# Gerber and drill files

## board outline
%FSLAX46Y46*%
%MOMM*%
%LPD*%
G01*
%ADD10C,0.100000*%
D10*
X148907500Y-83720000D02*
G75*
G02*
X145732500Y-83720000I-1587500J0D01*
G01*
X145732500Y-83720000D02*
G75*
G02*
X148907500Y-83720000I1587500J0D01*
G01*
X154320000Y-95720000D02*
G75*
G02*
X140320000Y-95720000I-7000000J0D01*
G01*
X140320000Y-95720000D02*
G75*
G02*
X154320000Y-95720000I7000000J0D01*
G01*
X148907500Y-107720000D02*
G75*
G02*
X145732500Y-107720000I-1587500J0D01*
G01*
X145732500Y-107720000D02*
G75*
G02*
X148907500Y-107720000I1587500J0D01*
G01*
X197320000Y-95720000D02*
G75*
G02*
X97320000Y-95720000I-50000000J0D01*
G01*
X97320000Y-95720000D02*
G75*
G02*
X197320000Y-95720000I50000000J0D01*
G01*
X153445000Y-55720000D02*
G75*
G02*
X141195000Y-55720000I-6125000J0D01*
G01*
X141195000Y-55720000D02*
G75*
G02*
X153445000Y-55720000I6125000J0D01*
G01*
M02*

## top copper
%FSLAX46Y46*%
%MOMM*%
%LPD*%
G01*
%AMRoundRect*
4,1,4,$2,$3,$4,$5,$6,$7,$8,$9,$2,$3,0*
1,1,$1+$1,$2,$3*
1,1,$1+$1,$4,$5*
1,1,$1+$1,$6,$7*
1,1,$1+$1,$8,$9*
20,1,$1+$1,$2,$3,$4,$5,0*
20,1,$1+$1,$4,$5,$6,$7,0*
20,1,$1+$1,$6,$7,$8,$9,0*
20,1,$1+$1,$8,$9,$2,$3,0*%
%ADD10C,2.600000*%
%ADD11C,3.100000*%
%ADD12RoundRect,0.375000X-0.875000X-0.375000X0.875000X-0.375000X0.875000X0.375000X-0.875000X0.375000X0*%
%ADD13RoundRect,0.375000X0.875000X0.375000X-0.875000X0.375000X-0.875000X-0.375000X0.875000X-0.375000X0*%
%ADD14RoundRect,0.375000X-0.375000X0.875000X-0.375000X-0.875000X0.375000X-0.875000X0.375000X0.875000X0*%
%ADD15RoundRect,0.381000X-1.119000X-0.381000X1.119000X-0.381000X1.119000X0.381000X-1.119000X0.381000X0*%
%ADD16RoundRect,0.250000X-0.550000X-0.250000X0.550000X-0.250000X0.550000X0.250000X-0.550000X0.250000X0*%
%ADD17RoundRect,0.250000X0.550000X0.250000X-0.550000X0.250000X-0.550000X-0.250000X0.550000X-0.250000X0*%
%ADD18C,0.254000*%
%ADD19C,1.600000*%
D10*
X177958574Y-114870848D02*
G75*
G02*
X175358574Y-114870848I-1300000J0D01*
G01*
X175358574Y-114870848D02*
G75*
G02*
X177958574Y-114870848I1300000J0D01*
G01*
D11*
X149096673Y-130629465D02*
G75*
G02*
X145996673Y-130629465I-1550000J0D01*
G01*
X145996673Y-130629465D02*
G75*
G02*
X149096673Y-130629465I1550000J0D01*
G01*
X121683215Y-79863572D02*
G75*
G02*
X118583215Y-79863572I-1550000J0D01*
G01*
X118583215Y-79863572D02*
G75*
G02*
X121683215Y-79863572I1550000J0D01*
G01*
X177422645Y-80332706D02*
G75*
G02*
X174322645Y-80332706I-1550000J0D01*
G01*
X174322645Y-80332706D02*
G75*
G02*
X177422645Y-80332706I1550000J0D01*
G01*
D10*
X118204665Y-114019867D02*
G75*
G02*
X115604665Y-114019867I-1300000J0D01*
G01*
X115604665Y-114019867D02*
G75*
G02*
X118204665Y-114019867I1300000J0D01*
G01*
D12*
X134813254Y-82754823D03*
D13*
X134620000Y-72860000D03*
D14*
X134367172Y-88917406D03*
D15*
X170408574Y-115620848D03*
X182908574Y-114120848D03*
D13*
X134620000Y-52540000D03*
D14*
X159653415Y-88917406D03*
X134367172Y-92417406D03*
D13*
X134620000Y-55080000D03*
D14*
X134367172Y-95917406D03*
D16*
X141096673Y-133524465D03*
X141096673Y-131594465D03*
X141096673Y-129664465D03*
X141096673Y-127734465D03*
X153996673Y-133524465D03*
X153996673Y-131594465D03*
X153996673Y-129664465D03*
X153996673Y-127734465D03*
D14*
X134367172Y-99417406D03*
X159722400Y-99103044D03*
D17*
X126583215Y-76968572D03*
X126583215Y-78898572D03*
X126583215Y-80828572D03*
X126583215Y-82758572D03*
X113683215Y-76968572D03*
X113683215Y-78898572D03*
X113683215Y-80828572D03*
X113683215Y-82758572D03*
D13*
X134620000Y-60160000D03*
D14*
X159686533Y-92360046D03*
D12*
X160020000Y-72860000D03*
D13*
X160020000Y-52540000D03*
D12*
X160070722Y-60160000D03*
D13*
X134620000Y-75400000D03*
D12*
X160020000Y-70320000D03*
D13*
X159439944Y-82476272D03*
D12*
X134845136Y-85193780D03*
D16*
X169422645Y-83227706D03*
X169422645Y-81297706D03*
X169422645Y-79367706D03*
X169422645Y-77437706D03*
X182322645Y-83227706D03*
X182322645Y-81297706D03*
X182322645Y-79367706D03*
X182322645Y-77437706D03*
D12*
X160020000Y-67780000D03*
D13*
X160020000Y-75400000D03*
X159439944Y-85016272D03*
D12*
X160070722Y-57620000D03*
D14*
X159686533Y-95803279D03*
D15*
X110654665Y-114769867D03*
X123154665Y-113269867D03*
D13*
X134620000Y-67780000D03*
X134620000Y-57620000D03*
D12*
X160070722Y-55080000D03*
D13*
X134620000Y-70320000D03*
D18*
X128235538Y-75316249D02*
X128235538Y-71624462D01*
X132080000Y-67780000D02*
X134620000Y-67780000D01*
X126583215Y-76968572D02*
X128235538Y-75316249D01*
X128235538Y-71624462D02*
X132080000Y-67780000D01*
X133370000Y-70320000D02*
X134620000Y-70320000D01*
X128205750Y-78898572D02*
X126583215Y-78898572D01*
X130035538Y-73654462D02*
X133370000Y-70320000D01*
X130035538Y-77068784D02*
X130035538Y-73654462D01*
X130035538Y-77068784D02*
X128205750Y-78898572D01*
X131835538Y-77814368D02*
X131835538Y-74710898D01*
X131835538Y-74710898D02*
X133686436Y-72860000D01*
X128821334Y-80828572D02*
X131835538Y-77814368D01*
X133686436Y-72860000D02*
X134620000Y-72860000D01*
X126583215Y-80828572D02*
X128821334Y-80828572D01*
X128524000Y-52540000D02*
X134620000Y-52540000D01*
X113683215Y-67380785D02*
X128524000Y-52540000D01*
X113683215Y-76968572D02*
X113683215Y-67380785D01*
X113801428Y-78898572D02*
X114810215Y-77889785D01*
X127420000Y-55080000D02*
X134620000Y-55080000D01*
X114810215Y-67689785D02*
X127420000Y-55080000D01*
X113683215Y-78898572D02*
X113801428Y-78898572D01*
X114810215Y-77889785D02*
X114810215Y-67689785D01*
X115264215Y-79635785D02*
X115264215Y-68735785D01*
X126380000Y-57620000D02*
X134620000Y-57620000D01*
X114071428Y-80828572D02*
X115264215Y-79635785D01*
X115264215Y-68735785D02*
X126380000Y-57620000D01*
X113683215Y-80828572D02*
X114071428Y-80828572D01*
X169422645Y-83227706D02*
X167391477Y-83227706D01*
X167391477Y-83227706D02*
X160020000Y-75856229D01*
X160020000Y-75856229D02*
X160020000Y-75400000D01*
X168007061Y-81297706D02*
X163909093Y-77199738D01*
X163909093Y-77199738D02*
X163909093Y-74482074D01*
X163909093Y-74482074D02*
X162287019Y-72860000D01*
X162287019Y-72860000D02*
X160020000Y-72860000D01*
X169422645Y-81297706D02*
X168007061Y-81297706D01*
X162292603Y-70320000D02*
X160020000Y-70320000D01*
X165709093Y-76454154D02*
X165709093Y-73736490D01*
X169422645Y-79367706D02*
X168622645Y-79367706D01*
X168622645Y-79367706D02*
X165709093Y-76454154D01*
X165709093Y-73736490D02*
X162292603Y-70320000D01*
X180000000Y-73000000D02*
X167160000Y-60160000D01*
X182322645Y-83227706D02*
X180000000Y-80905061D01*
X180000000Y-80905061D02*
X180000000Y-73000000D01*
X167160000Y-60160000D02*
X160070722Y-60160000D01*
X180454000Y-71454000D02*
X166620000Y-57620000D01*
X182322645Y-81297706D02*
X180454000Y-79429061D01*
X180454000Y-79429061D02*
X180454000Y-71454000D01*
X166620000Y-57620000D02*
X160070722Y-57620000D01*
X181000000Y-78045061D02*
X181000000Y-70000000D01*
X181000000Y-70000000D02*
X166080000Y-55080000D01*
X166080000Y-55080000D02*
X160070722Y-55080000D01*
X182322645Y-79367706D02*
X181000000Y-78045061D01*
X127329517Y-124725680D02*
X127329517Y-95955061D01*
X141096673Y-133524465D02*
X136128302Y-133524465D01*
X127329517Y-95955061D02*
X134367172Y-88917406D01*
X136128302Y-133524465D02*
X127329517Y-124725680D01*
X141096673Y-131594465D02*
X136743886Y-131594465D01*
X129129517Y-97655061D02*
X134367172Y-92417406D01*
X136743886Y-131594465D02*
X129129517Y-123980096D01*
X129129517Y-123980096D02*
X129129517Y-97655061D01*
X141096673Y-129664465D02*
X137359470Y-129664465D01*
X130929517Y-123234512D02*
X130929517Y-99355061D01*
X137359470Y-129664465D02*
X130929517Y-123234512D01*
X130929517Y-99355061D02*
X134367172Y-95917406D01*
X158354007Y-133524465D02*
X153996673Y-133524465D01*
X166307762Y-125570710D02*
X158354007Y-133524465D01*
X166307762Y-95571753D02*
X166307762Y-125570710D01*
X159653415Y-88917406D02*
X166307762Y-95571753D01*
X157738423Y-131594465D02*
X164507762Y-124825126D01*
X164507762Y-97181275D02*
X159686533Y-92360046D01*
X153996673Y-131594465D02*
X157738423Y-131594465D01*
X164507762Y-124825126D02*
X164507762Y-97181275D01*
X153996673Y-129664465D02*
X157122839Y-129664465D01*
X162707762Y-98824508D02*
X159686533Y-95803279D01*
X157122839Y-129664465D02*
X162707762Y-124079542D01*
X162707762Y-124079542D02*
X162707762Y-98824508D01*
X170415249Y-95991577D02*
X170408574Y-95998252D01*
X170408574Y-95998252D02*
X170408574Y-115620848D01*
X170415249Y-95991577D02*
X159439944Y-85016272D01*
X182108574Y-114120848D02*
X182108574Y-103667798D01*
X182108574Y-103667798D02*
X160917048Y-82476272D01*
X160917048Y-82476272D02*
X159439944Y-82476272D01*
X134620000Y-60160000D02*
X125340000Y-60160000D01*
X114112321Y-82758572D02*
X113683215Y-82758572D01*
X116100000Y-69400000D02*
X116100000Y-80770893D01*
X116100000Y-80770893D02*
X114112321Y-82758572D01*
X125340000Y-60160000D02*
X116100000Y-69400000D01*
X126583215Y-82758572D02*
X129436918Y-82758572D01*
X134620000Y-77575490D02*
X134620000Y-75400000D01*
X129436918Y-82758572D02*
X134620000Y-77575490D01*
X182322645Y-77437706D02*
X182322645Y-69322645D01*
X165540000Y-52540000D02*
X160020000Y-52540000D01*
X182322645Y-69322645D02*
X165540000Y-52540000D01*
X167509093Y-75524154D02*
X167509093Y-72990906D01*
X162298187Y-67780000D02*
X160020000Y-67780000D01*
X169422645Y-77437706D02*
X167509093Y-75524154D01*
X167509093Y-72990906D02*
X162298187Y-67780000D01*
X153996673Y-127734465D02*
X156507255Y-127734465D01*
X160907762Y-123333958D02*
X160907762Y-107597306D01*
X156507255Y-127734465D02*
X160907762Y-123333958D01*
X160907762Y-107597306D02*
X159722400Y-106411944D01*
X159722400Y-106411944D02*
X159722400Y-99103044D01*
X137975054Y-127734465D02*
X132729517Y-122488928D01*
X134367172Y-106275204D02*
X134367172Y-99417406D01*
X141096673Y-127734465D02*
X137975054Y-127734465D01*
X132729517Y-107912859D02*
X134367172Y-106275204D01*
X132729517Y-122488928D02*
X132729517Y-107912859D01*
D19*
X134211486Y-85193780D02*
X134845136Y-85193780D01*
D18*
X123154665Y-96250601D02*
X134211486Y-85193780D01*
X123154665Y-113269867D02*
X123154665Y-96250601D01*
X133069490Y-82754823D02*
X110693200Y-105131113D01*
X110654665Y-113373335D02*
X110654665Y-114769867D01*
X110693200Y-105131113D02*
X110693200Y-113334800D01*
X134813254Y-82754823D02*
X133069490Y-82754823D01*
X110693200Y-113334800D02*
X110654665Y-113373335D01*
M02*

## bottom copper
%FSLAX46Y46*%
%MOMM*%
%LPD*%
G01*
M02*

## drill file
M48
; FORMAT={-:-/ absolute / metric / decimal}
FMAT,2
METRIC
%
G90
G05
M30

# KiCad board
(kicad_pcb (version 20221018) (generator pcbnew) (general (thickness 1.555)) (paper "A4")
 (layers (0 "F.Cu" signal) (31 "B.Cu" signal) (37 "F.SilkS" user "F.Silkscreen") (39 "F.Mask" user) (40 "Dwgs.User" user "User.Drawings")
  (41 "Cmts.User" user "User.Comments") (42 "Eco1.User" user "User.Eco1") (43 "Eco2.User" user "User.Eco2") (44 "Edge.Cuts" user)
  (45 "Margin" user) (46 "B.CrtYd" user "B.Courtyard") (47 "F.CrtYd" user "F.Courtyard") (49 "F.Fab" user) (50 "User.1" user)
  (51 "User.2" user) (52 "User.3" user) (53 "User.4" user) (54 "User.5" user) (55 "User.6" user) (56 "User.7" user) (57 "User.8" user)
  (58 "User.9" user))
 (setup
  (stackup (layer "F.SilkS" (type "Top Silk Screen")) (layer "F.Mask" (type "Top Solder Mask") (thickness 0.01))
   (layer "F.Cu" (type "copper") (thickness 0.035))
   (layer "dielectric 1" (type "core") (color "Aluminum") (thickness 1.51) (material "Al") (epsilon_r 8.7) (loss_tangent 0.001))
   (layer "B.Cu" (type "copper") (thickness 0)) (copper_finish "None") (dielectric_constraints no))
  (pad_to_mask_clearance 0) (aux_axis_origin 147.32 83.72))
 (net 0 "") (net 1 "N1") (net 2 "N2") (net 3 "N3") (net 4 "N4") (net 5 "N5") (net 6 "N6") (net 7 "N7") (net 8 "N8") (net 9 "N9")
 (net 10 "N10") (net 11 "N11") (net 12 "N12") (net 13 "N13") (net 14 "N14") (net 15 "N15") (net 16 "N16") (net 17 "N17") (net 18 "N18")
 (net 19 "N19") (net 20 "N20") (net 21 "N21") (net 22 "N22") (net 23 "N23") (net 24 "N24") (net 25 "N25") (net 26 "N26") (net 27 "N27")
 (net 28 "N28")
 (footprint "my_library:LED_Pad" (layer "F.Cu") (at 134.813254 85.294823)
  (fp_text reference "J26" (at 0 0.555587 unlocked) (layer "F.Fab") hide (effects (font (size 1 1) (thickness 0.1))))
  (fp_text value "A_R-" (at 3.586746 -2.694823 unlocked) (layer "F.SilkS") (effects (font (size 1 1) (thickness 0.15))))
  (pad "1" smd roundrect (at 0 -2.54) (size 2.5 1.5) (layers "F.Cu" "F.Mask") (roundrect_rratio 0.25) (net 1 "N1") (thermal_bridge_angle 45)))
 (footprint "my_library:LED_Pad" (layer "F.Cu") (at 134.62 70.32 180)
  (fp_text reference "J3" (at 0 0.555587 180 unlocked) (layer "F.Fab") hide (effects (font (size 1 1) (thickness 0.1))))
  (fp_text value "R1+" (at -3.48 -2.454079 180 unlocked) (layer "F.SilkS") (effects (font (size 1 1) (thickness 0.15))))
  (pad "1" smd roundrect (at 0 -2.54 180) (size 2.5 1.5) (layers "F.Cu" "F.Mask") (roundrect_rratio 0.25) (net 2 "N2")
   (thermal_bridge_angle 45)))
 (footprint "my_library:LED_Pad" (layer "F.Cu") (at 131.827172 88.917406 -90)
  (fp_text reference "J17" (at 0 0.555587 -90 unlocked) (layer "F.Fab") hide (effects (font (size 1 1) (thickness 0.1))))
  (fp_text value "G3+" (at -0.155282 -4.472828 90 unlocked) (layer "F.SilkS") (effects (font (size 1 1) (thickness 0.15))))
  (pad "1" smd roundrect (at 0 -2.54 270) (size 2.5 1.5) (layers "F.Cu" "F.Mask") (roundrect_rratio 0.25) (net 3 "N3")
   (thermal_bridge_angle 45)))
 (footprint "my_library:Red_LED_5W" (layer "F.Cu") (at 177.028574 114.120848)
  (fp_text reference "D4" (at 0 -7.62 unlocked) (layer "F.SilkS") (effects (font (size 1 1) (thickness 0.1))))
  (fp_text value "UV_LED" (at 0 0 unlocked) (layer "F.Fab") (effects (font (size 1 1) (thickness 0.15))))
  (fp_circle (center -0.37 0.75) (end 2.13 0.75) (stroke (width 0.2) (type solid)) (fill solid) (layer "F.Cu"))
  (pad "1" smd roundrect (at -6.62 1.5) (size 3 1.524) (layers "F.Cu" "F.Paste" "F.Mask") (roundrect_rratio 0.25) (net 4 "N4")
   (thermal_bridge_angle 45))
  (pad "2" smd roundrect (at 5.88 0) (size 3 1.524) (layers "F.Cu" "F.Paste" "F.Mask") (roundrect_rratio 0.25) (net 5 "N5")
   (thermal_bridge_angle 45)))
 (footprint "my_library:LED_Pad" (layer "F.Cu") (at 134.62 50 180)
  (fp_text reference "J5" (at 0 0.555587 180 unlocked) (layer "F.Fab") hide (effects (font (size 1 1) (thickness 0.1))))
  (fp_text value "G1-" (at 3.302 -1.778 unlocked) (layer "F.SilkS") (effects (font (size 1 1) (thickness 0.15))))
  (pad "1" smd roundrect (at 0 -2.54 180) (size 2.5 1.5) (layers "F.Cu" "F.Mask") (roundrect_rratio 0.25) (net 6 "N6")
   (thermal_bridge_angle 45)))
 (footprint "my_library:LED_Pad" (layer "F.Cu") (at 157.113415 88.917406 -90)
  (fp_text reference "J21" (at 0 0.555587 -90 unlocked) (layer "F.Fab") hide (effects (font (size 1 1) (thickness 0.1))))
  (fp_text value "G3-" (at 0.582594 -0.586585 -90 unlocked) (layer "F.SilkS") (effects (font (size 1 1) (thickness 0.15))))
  (pad "1" smd roundrect (at 0 -2.54 270) (size 2.5 1.5) (layers "F.Cu" "F.Mask") (roundrect_rratio 0.25) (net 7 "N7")
   (thermal_bridge_angle 45)))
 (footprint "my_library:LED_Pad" (layer "F.Cu") (at 131.827172 92.417406 -90)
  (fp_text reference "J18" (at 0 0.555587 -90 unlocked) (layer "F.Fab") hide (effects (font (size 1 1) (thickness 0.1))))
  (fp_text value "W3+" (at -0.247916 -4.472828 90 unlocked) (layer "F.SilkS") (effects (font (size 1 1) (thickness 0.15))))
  (pad "1" smd roundrect (at 0 -2.54 270) (size 2.5 1.5) (layers "F.Cu" "F.Mask") (roundrect_rratio 0.25) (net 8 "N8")
   (thermal_bridge_angle 45)))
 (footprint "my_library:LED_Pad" (layer "F.Cu") (at 134.62 52.54 180)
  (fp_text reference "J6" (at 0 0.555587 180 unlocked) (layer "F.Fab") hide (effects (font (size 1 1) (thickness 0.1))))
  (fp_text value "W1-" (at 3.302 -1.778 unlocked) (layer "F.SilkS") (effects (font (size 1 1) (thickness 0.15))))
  (pad "1" smd roundrect (at 0 -2.54 180) (size 2.5 1.5) (layers "F.Cu" "F.Mask") (roundrect_rratio 0.25) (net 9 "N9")
   (thermal_bridge_angle 45)))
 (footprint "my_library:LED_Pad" (layer "F.Cu") (at 131.827172 95.917406 -90)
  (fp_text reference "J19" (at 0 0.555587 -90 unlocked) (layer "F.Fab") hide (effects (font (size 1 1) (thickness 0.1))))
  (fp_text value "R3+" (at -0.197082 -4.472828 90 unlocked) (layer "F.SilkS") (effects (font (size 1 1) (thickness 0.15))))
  (pad "1" smd roundrect (at 0 -2.54 270) (size 2.5 1.5) (layers "F.Cu" "F.Mask") (roundrect_rratio 0.25) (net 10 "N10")
   (thermal_bridge_angle 45)))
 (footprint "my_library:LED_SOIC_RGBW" (layer "F.Cu") (at 145.916673 139.214465)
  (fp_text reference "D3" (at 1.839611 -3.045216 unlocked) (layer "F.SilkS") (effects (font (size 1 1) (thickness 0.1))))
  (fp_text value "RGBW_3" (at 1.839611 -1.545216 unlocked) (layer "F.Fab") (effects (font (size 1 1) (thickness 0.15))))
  (fp_circle (center 1.63 -8.585) (end 4.63 -8.585) (stroke (width 0.2) (type solid)) (fill solid) (layer "F.Cu"))
  (pad "1" smd roundrect (at -4.82 -5.69) (size 1.6 1) (layers "F.Cu" "F.Mask") (roundrect_rratio 0.25) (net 3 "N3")
   (thermal_bridge_angle 45))
  (pad "2" smd roundrect (at -4.82 -7.62) (size 1.6 1) (layers "F.Cu" "F.Mask") (roundrect_rratio 0.25) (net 8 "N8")
   (thermal_bridge_angle 45))
  (pad "3" smd roundrect (at -4.82 -9.55) (size 1.6 1) (layers "F.Cu" "F.Mask") (roundrect_rratio 0.25) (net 10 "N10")
   (thermal_bridge_angle 45))
  (pad "4" smd roundrect (at -4.82 -11.48) (size 1.6 1) (layers "F.Cu" "F.Mask") (roundrect_rratio 0.25) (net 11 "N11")
   (thermal_bridge_angle 45))
  (pad "5" smd roundrect (at 8.08 -5.69) (size 1.6 1) (layers "F.Cu" "F.Mask") (roundrect_rratio 0.25) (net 7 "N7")
   (thermal_bridge_angle 45))
  (pad "6" smd roundrect (at 8.08 -7.62) (size 1.6 1) (layers "F.Cu" "F.Mask") (roundrect_rratio 0.25) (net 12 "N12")
   (thermal_bridge_angle 45))
  (pad "7" smd roundrect (at 8.08 -9.55) (size 1.6 1) (layers "F.Cu" "F.Mask") (roundrect_rratio 0.25) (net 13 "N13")
   (thermal_bridge_angle 45))
  (pad "8" smd roundrect (at 8.08 -11.48) (size 1.6 1) (layers "F.Cu" "F.Mask") (roundrect_rratio 0.25) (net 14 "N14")
   (thermal_bridge_angle 45)))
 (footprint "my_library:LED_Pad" (layer "F.Cu") (at 131.827172 99.417406 -90)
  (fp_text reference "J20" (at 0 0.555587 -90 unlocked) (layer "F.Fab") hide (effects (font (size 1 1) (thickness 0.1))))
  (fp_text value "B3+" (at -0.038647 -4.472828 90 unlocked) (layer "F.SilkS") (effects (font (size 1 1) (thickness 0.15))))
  (pad "1" smd roundrect (at 0 -2.54 270) (size 2.5 1.5) (layers "F.Cu" "F.Mask") (roundrect_rratio 0.25) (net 11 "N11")
   (thermal_bridge_angle 45)))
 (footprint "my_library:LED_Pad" (layer "F.Cu") (at 157.1824 99.103044 -90)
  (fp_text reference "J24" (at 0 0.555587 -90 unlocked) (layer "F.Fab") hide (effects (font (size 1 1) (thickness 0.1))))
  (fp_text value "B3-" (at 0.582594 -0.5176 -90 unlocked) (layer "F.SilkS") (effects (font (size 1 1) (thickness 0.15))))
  (pad "1" smd roundrect (at 0 -2.54 270) (size 2.5 1.5) (layers "F.Cu" "F.Mask") (roundrect_rratio 0.25) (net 14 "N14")
   (thermal_bridge_angle 45)))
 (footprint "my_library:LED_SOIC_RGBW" (layer "F.Cu") (at 121.763215 71.278572 180)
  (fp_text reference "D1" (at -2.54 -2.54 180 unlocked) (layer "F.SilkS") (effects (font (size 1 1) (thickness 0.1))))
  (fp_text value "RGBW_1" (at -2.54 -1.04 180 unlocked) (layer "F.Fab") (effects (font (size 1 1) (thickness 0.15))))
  (fp_circle (center 1.63 -8.585) (end 4.63 -8.585) (stroke (width 0.2) (type solid)) (fill solid) (layer "F.Cu"))
  (pad "1" smd roundrect (at -4.82 -5.69 180) (size 1.6 1) (layers "F.Cu" "F.Mask") (roundrect_rratio 0.25) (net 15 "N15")
   (thermal_bridge_angle 45))
  (pad "2" smd roundrect (at -4.82 -7.62 180) (size 1.6 1) (layers "F.Cu" "F.Mask") (roundrect_rratio 0.25) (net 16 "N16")
   (thermal_bridge_angle 45))
  (pad "3" smd roundrect (at -4.82 -9.55 180) (size 1.6 1) (layers "F.Cu" "F.Mask") (roundrect_rratio 0.25) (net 2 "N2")
   (thermal_bridge_angle 45))
  (pad "4" smd roundrect (at -4.82 -11.48 180) (size 1.6 1) (layers "F.Cu" "F.Mask") (roundrect_rratio 0.25) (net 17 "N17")
   (thermal_bridge_angle 45))
  (pad "5" smd roundrect (at 8.08 -5.69 180) (size 1.6 1) (layers "F.Cu" "F.Mask") (roundrect_rratio 0.25) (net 6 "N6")
   (thermal_bridge_angle 45))
  (pad "6" smd roundrect (at 8.08 -7.62 180) (size 1.6 1) (layers "F.Cu" "F.Mask") (roundrect_rratio 0.25) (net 9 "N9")
   (thermal_bridge_angle 45))
  (pad "7" smd roundrect (at 8.08 -9.55 180) (size 1.6 1) (layers "F.Cu" "F.Mask") (roundrect_rratio 0.25) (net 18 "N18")
   (thermal_bridge_angle 45))
  (pad "8" smd roundrect (at 8.08 -11.48 180) (size 1.6 1) (layers "F.Cu" "F.Mask") (roundrect_rratio 0.25) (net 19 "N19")
   (thermal_bridge_angle 45)))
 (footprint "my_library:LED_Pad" (layer "F.Cu") (at 134.62 57.62 180)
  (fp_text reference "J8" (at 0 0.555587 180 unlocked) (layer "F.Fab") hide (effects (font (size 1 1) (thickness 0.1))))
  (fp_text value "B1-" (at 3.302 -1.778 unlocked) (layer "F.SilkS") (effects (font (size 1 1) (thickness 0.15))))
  (pad "1" smd roundrect (at 0 -2.54 180) (size 2.5 1.5) (layers "F.Cu" "F.Mask") (roundrect_rratio 0.25) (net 19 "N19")
   (thermal_bridge_angle 45)))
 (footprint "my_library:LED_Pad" (layer "F.Cu") (at 157.146533 92.360046 -90)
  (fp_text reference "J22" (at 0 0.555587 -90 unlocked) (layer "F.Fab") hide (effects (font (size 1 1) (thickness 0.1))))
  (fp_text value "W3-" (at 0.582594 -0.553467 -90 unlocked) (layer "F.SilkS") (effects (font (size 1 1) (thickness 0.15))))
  (pad "1" smd roundrect (at 0 -2.54 270) (size 2.5 1.5) (layers "F.Cu" "F.Mask") (roundrect_rratio 0.25) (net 12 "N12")
   (thermal_bridge_angle 45)))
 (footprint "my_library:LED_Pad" (layer "F.Cu") (at 160.02 75.4)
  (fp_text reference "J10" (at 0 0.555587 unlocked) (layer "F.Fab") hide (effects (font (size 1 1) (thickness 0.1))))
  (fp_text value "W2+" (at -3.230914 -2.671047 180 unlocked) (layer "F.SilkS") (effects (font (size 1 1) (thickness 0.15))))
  (pad "1" smd roundrect (at 0 -2.54) (size 2.5 1.5) (layers "F.Cu" "F.Mask") (roundrect_rratio 0.25) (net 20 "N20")
   (thermal_bridge_angle 45)))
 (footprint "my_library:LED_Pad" (layer "F.Cu") (at 160.02 50 180)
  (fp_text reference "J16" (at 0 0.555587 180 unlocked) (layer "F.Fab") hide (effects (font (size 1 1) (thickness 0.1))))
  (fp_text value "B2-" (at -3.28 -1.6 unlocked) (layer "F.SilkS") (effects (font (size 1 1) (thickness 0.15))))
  (pad "1" smd roundrect (at 0 -2.54 180) (size 2.5 1.5) (layers "F.Cu" "F.Mask") (roundrect_rratio 0.25) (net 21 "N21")
   (thermal_bridge_angle 45)))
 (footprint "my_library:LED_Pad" (layer "F.Cu") (at 160.070722 62.7)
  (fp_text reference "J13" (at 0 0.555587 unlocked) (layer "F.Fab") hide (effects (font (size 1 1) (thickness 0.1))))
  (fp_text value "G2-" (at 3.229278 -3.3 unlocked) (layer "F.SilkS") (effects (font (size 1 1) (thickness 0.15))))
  (pad "1" smd roundrect (at 0 -2.54) (size 2.5 1.5) (layers "F.Cu" "F.Mask") (roundrect_rratio 0.25) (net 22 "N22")
   (thermal_bridge_angle 45)))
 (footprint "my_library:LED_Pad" (layer "F.Cu") (at 134.62 72.86 180)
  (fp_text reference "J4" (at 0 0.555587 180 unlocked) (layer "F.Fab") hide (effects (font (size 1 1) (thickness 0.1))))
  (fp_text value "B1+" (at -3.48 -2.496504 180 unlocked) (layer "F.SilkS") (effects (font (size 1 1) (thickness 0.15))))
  (pad "1" smd roundrect (at 0 -2.54 180) (size 2.5 1.5) (layers "F.Cu" "F.Mask") (roundrect_rratio 0.25) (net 17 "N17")
   (thermal_bridge_angle 45)))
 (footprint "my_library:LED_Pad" (layer "F.Cu") (at 160.02 72.86)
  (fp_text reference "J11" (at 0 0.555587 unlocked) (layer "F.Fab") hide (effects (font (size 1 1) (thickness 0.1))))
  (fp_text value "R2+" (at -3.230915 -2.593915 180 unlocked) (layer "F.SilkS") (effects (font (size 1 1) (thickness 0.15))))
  (pad "1" smd roundrect (at 0 -2.54) (size 2.5 1.5) (layers "F.Cu" "F.Mask") (roundrect_rratio 0.25) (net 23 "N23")
   (thermal_bridge_angle 45)))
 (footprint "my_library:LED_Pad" (layer "F.Cu") (at 159.439944 79.936272 180)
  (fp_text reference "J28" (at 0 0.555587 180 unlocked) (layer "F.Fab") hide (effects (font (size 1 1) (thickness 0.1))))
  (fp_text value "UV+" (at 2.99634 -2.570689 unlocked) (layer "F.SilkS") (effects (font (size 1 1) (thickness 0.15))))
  (pad "1" smd roundrect (at 0 -2.54 180) (size 2.5 1.5) (layers "F.Cu" "F.Mask") (roundrect_rratio 0.25) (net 5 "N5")
   (thermal_bridge_angle 45)))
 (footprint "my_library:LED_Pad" (layer "F.Cu") (at 134.845136 87.73378)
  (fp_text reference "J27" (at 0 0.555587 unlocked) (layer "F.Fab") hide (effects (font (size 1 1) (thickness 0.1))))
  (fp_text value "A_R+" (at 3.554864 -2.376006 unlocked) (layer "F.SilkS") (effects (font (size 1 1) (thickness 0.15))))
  (pad "1" smd roundrect (at 0 -2.54) (size 2.5 1.5) (layers "F.Cu" "F.Mask") (roundrect_rratio 0.25) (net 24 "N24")
   (thermal_bridge_angle 45)))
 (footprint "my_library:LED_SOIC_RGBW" (layer "F.Cu") (at 174.242645 88.917706)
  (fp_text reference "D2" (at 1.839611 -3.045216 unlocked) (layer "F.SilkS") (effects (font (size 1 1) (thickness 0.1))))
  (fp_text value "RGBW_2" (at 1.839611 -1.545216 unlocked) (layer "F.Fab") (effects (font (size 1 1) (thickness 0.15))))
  (fp_circle (center 1.63 -8.585) (end 4.63 -8.585) (stroke (width 0.2) (type solid)) (fill solid) (layer "F.Cu"))
  (pad "1" smd roundrect (at -4.82 -5.69) (size 1.6 1) (layers "F.Cu" "F.Mask") (roundrect_rratio 0.25) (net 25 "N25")
   (thermal_bridge_angle 45))
  (pad "2" smd roundrect (at -4.82 -7.62) (size 1.6 1) (layers "F.Cu" "F.Mask") (roundrect_rratio 0.25) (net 20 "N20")
   (thermal_bridge_angle 45))
  (pad "3" smd roundrect (at -4.82 -9.55) (size 1.6 1) (layers "F.Cu" "F.Mask") (roundrect_rratio 0.25) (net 23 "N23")
   (thermal_bridge_angle 45))
  (pad "4" smd roundrect (at -4.82 -11.48) (size 1.6 1) (layers "F.Cu" "F.Mask") (roundrect_rratio 0.25) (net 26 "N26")
   (thermal_bridge_angle 45))
  (pad "5" smd roundrect (at 8.08 -5.69) (size 1.6 1) (layers "F.Cu" "F.Mask") (roundrect_rratio 0.25) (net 22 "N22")
   (thermal_bridge_angle 45))
  (pad "6" smd roundrect (at 8.08 -7.62) (size 1.6 1) (layers "F.Cu" "F.Mask") (roundrect_rratio 0.25) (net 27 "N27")
   (thermal_bridge_angle 45))
  (pad "7" smd roundrect (at 8.08 -9.55) (size 1.6 1) (layers "F.Cu" "F.Mask") (roundrect_rratio 0.25) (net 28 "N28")
   (thermal_bridge_angle 45))
  (pad "8" smd roundrect (at 8.08 -11.48) (size 1.6 1) (layers "F.Cu" "F.Mask") (roundrect_rratio 0.25) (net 21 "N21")
   (thermal_bridge_angle 45)))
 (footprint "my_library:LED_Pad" (layer "F.Cu") (at 160.02 70.32)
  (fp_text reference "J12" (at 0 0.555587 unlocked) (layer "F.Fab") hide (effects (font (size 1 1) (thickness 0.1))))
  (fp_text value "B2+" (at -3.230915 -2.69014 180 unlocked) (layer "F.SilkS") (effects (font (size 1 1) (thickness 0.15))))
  (pad "1" smd roundrect (at 0 -2.54) (size 2.5 1.5) (layers "F.Cu" "F.Mask") (roundrect_rratio 0.25) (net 26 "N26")
   (thermal_bridge_angle 45)))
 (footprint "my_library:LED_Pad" (layer "F.Cu") (at 160.02 72.86 180)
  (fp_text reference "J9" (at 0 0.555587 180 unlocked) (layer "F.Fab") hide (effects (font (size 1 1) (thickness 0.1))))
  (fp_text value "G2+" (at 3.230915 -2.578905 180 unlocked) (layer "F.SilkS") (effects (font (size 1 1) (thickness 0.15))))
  (pad "1" smd roundrect (at 0 -2.54 180) (size 2.5 1.5) (layers "F.Cu" "F.Mask") (roundrect_rratio 0.25) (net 25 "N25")
   (thermal_bridge_angle 45)))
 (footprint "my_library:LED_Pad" (layer "F.Cu") (at 159.439944 82.476272 180)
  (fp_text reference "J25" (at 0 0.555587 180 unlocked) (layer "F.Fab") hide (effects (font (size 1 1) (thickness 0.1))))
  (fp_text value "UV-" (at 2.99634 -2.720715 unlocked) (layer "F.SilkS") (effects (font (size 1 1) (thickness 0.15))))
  (pad "1" smd roundrect (at 0 -2.54 180) (size 2.5 1.5) (layers "F.Cu" "F.Mask") (roundrect_rratio 0.25) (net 4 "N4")
   (thermal_bridge_angle 45)))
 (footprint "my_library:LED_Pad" (layer "F.Cu") (at 160.070722 60.16)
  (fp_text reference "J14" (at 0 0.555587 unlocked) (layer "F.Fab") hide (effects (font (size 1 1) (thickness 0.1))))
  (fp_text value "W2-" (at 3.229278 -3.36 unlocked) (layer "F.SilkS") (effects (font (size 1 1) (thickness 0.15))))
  (pad "1" smd roundrect (at 0 -2.54) (size 2.5 1.5) (layers "F.Cu" "F.Mask") (roundrect_rratio 0.25) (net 27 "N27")
   (thermal_bridge_angle 45)))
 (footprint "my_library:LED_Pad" (layer "F.Cu") (at 157.146533 95.803279 -90)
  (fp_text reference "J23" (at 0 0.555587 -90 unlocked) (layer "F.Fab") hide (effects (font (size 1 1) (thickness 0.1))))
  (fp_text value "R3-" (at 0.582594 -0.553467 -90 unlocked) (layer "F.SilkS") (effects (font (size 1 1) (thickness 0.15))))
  (pad "1" smd roundrect (at 0 -2.54 270) (size 2.5 1.5) (layers "F.Cu" "F.Mask") (roundrect_rratio 0.25) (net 13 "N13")
   (thermal_bridge_angle 45)))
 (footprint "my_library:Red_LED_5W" (layer "F.Cu") (at 117.274665 113.269867)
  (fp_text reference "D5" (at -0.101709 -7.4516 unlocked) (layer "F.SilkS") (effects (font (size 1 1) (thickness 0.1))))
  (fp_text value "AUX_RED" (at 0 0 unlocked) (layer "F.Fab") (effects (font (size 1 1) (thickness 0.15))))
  (fp_circle (center -0.37 0.75) (end 2.13 0.75) (stroke (width 0.2) (type solid)) (fill solid) (layer "F.Cu"))
  (pad "1" smd roundrect (at -6.62 1.5) (size 3 1.524) (layers "F.Cu" "F.Paste" "F.Mask") (roundrect_rratio 0.25) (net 1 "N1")
   (thermal_bridge_angle 45))
  (pad "2" smd roundrect (at 5.88 0) (size 3 1.524) (layers "F.Cu" "F.Paste" "F.Mask") (roundrect_rratio 0.25) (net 24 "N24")
   (thermal_bridge_angle 45)))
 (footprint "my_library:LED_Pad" (layer "F.Cu") (at 134.62 65.24 180)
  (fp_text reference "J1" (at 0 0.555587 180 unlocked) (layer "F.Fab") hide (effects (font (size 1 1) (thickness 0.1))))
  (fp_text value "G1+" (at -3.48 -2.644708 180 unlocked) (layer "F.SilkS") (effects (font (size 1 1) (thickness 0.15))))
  (pad "1" smd roundrect (at 0 -2.54 180) (size 2.5 1.5) (layers "F.Cu" "F.Mask") (roundrect_rratio 0.25) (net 15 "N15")
   (thermal_bridge_angle 45)))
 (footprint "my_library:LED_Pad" (layer "F.Cu") (at 134.62 55.08 180)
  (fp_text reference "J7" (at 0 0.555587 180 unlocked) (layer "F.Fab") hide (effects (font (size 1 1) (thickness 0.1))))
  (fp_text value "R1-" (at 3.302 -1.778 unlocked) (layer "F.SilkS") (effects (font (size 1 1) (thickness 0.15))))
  (pad "1" smd roundrect (at 0 -2.54 180) (size 2.5 1.5) (layers "F.Cu" "F.Mask") (roundrect_rratio 0.25) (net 18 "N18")
   (thermal_bridge_angle 45)))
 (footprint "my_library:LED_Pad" (layer "F.Cu") (at 160.070722 57.62)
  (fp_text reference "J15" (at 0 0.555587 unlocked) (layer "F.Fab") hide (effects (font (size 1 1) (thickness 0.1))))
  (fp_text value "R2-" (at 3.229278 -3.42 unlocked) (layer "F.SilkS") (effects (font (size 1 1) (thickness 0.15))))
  (pad "1" smd roundrect (at 0 -2.54) (size 2.5 1.5) (layers "F.Cu" "F.Mask") (roundrect_rratio 0.25) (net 28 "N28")
   (thermal_bridge_angle 45)))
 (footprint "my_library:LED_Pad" (layer "F.Cu") (at 134.62 67.78 180)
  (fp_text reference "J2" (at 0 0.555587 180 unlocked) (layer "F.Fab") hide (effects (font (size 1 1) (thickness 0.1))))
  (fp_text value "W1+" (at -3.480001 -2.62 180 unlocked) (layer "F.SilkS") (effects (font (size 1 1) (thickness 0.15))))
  (pad "1" smd roundrect (at 0 -2.54 180) (size 2.5 1.5) (layers "F.Cu" "F.Mask") (roundrect_rratio 0.25) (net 16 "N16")
   (thermal_bridge_angle 45)))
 (gr_circle locked (center 147.32 83.72) (end 148.9075 83.72) (stroke (width 0.1) (type default)) (fill none) (layer "Edge.Cuts"))
 (gr_circle locked (center 147.32 95.72) (end 154.32 95.72) (stroke (width 0.1) (type default)) (fill none) (layer "Edge.Cuts"))
 (gr_circle locked (center 147.32 107.72) (end 148.9075 107.72) (stroke (width 0.1) (type default)) (fill none) (layer "Edge.Cuts"))
 (gr_circle locked (center 147.32 95.72) (end 197.32 95.72) (stroke (width 0.1) (type default)) (fill none) (layer "Edge.Cuts"))
 (gr_circle locked (center 147.32 55.72) (end 153.445 55.72) (stroke (width 0.1) (type default)) (fill none) (layer "Edge.Cuts"))
 (segment (start 128.235538 75.316249) (end 128.235538 71.624462) (width 0.254) (layer "F.Cu") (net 15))
 (segment (start 132.08 67.78) (end 134.62 67.78) (width 0.254) (layer "F.Cu") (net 15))
 (segment (start 126.583215 76.968572) (end 128.235538 75.316249) (width 0.254) (layer "F.Cu") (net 15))
 (segment (start 128.235538 71.624462) (end 132.08 67.78) (width 0.254) (layer "F.Cu") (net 15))
 (segment (start 133.37 70.32) (end 134.62 70.32) (width 0.254) (layer "F.Cu") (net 16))
 (segment (start 128.20575 78.898572) (end 126.583215 78.898572) (width 0.254) (layer "F.Cu") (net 16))
 (segment (start 130.035538 73.654462) (end 133.37 70.32) (width 0.254) (layer "F.Cu") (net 16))
 (segment (start 130.035538 77.068784) (end 130.035538 73.654462) (width 0.254) (layer "F.Cu") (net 16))
 (segment (start 130.035538 77.068784) (end 128.20575 78.898572) (width 0.254) (layer "F.Cu") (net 16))
 (segment (start 131.835538 77.814368) (end 131.835538 74.710898) (width 0.254) (layer "F.Cu") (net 2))
 (segment (start 131.835538 74.710898) (end 133.686436 72.86) (width 0.254) (layer "F.Cu") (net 2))
 (segment (start 128.821334 80.828572) (end 131.835538 77.814368) (width 0.254) (layer "F.Cu") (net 2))
 (segment (start 133.686436 72.86) (end 134.62 72.86) (width 0.254) (layer "F.Cu") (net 2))
 (segment (start 126.583215 80.828572) (end 128.821334 80.828572) (width 0.254) (layer "F.Cu") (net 2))
 (segment (start 128.524 52.54) (end 134.62 52.54) (width 0.254) (layer "F.Cu") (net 6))
 (segment (start 113.683215 67.380785) (end 128.524 52.54) (width 0.254) (layer "F.Cu") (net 6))
 (segment (start 113.683215 76.968572) (end 113.683215 67.380785) (width 0.254) (layer "F.Cu") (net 6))
 (segment (start 113.801428 78.898572) (end 114.810215 77.889785) (width 0.254) (layer "F.Cu") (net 9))
 (segment (start 127.42 55.08) (end 134.62 55.08) (width 0.254) (layer "F.Cu") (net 9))
 (segment (start 114.810215 67.689785) (end 127.42 55.08) (width 0.254) (layer "F.Cu") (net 9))
 (segment (start 113.683215 78.898572) (end 113.801428 78.898572) (width 0.254) (layer "F.Cu") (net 9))
 (segment (start 114.810215 77.889785) (end 114.810215 67.689785) (width 0.254) (layer "F.Cu") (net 9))
 (segment (start 115.264215 79.635785) (end 115.264215 68.735785) (width 0.254) (layer "F.Cu") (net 18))
 (segment (start 126.38 57.62) (end 134.62 57.62) (width 0.254) (layer "F.Cu") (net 18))
 (segment (start 114.071428 80.828572) (end 115.264215 79.635785) (width 0.254) (layer "F.Cu") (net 18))
 (segment (start 115.264215 68.735785) (end 126.38 57.62) (width 0.254) (layer "F.Cu") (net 18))
 (segment (start 113.683215 80.828572) (end 114.071428 80.828572) (width 0.254) (layer "F.Cu") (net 18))
 (segment (start 169.422645 83.227706) (end 167.391477 83.227706) (width 0.254) (layer "F.Cu") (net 25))
 (segment (start 167.391477 83.227706) (end 160.02 75.856229) (width 0.254) (layer "F.Cu") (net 25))
 (segment (start 160.02 75.856229) (end 160.02 75.4) (width 0.254) (layer "F.Cu") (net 25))
 (segment (start 168.007061 81.297706) (end 163.909093 77.199738) (width 0.254) (layer "F.Cu") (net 20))
 (segment (start 163.909093 77.199738) (end 163.909093 74.482074) (width 0.254) (layer "F.Cu") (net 20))
 (segment (start 163.909093 74.482074) (end 162.287019 72.86) (width 0.254) (layer "F.Cu") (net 20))
 (segment (start 162.287019 72.86) (end 160.02 72.86) (width 0.254) (layer "F.Cu") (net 20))
 (segment (start 169.422645 81.297706) (end 168.007061 81.297706) (width 0.254) (layer "F.Cu") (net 20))
 (segment (start 162.292603 70.32) (end 160.02 70.32) (width 0.254) (layer "F.Cu") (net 23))
 (segment (start 165.709093 76.454154) (end 165.709093 73.73649) (width 0.254) (layer "F.Cu") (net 23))
 (segment (start 169.422645 79.367706) (end 168.622645 79.367706) (width 0.254) (layer "F.Cu") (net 23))
 (segment (start 168.622645 79.367706) (end 165.709093 76.454154) (width 0.254) (layer "F.Cu") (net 23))
 (segment (start 165.709093 73.73649) (end 162.292603 70.32) (width 0.254) (layer "F.Cu") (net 23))
 (segment (start 180 73) (end 167.16 60.16) (width 0.254) (layer "F.Cu") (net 22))
 (segment (start 182.322645 83.227706) (end 180 80.905061) (width 0.254) (layer "F.Cu") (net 22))
 (segment (start 180 80.905061) (end 180 73) (width 0.254) (layer "F.Cu") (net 22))
 (segment (start 167.16 60.16) (end 160.070722 60.16) (width 0.254) (layer "F.Cu") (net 22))
 (segment (start 180.454 71.454) (end 166.62 57.62) (width 0.254) (layer "F.Cu") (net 27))
 (segment (start 182.322645 81.297706) (end 180.454 79.429061) (width 0.254) (layer "F.Cu") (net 27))
 (segment (start 180.454 79.429061) (end 180.454 71.454) (width 0.254) (layer "F.Cu") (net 27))
 (segment (start 166.62 57.62) (end 160.070722 57.62) (width 0.254) (layer "F.Cu") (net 27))
 (segment (start 181 78.045061) (end 181 70) (width 0.254) (layer "F.Cu") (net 28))
 (segment (start 181 70) (end 166.08 55.08) (width 0.254) (layer "F.Cu") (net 28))
 (segment (start 166.08 55.08) (end 160.070722 55.08) (width 0.254) (layer "F.Cu") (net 28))
 (segment (start 182.322645 79.367706) (end 181 78.045061) (width 0.254) (layer "F.Cu") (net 28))
 (segment (start 127.329517 124.72568) (end 127.329517 95.955061) (width 0.254) (layer "F.Cu") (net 3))
 (segment (start 141.096673 133.524465) (end 136.128302 133.524465) (width 0.254) (layer "F.Cu") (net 3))
 (segment (start 127.329517 95.955061) (end 134.367172 88.917406) (width 0.254) (layer "F.Cu") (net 3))
 (segment (start 136.128302 133.524465) (end 127.329517 124.72568) (width 0.254) (layer "F.Cu") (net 3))
 (segment (start 141.096673 131.594465) (end 136.743886 131.594465) (width 0.254) (layer "F.Cu") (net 8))
 (segment (start 129.129517 97.655061) (end 134.367172 92.417406) (width 0.254) (layer "F.Cu") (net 8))
 (segment (start 136.743886 131.594465) (end 129.129517 123.980096) (width 0.254) (layer "F.Cu") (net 8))
 (segment (start 129.129517 123.980096) (end 129.129517 97.655061) (width 0.254) (layer "F.Cu") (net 8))
 (segment (start 141.096673 129.664465) (end 137.35947 129.664465) (width 0.254) (layer "F.Cu") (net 10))
 (segment (start 130.929517 123.234512) (end 130.929517 99.355061) (width 0.254) (layer "F.Cu") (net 10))
 (segment (start 137.35947 129.664465) (end 130.929517 123.234512) (width 0.254) (layer "F.Cu") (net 10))
 (segment (start 130.929517 99.355061) (end 134.367172 95.917406) (width 0.254) (layer "F.Cu") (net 10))
 (segment (start 158.354007 133.524465) (end 153.996673 133.524465) (width 0.254) (layer "F.Cu") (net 7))
 (segment (start 166.307762 125.57071) (end 158.354007 133.524465) (width 0.254) (layer "F.Cu") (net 7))
 (segment (start 166.307762 95.571753) (end 166.307762 125.57071) (width 0.254) (layer "F.Cu") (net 7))
 (segment (start 159.653415 88.917406) (end 166.307762 95.571753) (width 0.254) (layer "F.Cu") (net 7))
 (segment (start 157.738423 131.594465) (end 164.507762 124.825126) (width 0.254) (layer "F.Cu") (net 12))
 (segment (start 164.507762 97.181275) (end 159.686533 92.360046) (width 0.254) (layer "F.Cu") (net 12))
 (segment (start 153.996673 131.594465) (end 157.738423 131.594465) (width 0.254) (layer "F.Cu") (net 12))
 (segment (start 164.507762 124.825126) (end 164.507762 97.181275) (width 0.254) (layer "F.Cu") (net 12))
 (segment (start 153.996673 129.664465) (end 157.122839 129.664465) (width 0.254) (layer "F.Cu") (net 13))
 (segment (start 162.707762 98.824508) (end 159.686533 95.803279) (width 0.254) (layer "F.Cu") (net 13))
 (segment (start 157.122839 129.664465) (end 162.707762 124.079542) (width 0.254) (layer "F.Cu") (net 13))
 (segment (start 162.707762 124.079542) (end 162.707762 98.824508) (width 0.254) (layer "F.Cu") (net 13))
 (segment (start 170.415249 95.991577) (end 170.408574 95.998252) (width 0.254) (layer "F.Cu") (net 4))
 (segment (start 170.408574 95.998252) (end 170.408574 115.620848) (width 0.254) (layer "F.Cu") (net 4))
 (segment (start 170.415249 95.991577) (end 159.439944 85.016272) (width 0.254) (layer "F.Cu") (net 4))
 (segment (start 182.108574 114.120848) (end 182.108574 103.667798) (width 0.254) (layer "F.Cu") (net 5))
 (segment (start 182.108574 103.667798) (end 160.917048 82.476272) (width 0.254) (layer "F.Cu") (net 5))
 (segment (start 160.917048 82.476272) (end 159.439944 82.476272) (width 0.254) (layer "F.Cu") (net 5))
 (segment (start 134.62 60.16) (end 125.34 60.16) (width 0.254) (layer "F.Cu") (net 19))
 (segment (start 114.112321 82.758572) (end 113.683215 82.758572) (width 0.254) (layer "F.Cu") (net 19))
 (segment (start 116.1 69.4) (end 116.1 80.770893) (width 0.254) (layer "F.Cu") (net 19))
 (segment (start 116.1 80.770893) (end 114.112321 82.758572) (width 0.254) (layer "F.Cu") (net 19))
 (segment (start 125.34 60.16) (end 116.1 69.4) (width 0.254) (layer "F.Cu") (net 19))
 (segment (start 126.583215 82.758572) (end 129.436918 82.758572) (width 0.254) (layer "F.Cu") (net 17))
 (segment (start 134.62 77.57549) (end 134.62 75.4) (width 0.254) (layer "F.Cu") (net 17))
 (segment (start 129.436918 82.758572) (end 134.62 77.57549) (width 0.254) (layer "F.Cu") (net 17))
 (segment (start 182.322645 77.437706) (end 182.322645 69.322645) (width 0.254) (layer "F.Cu") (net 21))
 (segment (start 165.54 52.54) (end 160.02 52.54) (width 0.254) (layer "F.Cu") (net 21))
 (segment (start 182.322645 69.322645) (end 165.54 52.54) (width 0.254) (layer "F.Cu") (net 21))
 (segment (start 167.509093 75.524154) (end 167.509093 72.990906) (width 0.254) (layer "F.Cu") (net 26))
 (segment (start 162.298187 67.78) (end 160.02 67.78) (width 0.254) (layer "F.Cu") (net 26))
 (segment (start 169.422645 77.437706) (end 167.509093 75.524154) (width 0.254) (layer "F.Cu") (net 26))
 (segment (start 167.509093 72.990906) (end 162.298187 67.78) (width 0.254) (layer "F.Cu") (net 26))
 (segment (start 153.996673 127.734465) (end 156.507255 127.734465) (width 0.254) (layer "F.Cu") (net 14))
 (segment (start 160.907762 123.333958) (end 160.907762 107.597306) (width 0.254) (layer "F.Cu") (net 14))
 (segment (start 156.507255 127.734465) (end 160.907762 123.333958) (width 0.254) (layer "F.Cu") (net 14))
 (segment (start 160.907762 107.597306) (end 159.7224 106.411944) (width 0.254) (layer "F.Cu") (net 14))
 (segment (start 159.7224 106.411944) (end 159.7224 99.103044) (width 0.254) (layer "F.Cu") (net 14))
 (segment (start 137.975054 127.734465) (end 132.729517 122.488928) (width 0.254) (layer "F.Cu") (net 11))
 (segment (start 134.367172 106.275204) (end 134.367172 99.417406) (width 0.254) (layer "F.Cu") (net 11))
 (segment (start 141.096673 127.734465) (end 137.975054 127.734465) (width 0.254) (layer "F.Cu") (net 11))
 (segment (start 132.729517 107.912859) (end 134.367172 106.275204) (width 0.254) (layer "F.Cu") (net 11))
 (segment (start 132.729517 122.488928) (end 132.729517 107.912859) (width 0.254) (layer "F.Cu") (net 11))
 (segment (start 134.211486 85.19378) (end 134.845136 85.19378) (width 1.6) (layer "F.Cu") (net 24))
 (segment (start 123.154665 96.250601) (end 134.211486 85.19378) (width 0.254) (layer "F.Cu") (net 24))
 (segment (start 123.154665 113.269867) (end 123.154665 96.250601) (width 0.254) (layer "F.Cu") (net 24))
 (segment (start 133.06949 82.754823) (end 110.6932 105.131113) (width 0.254) (layer "F.Cu") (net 1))
 (segment (start 110.654665 113.373335) (end 110.654665 114.769867) (width 0.254) (layer "F.Cu") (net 1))
 (segment (start 110.6932 105.131113) (end 110.6932 113.3348) (width 0.254) (layer "F.Cu") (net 1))
 (segment (start 134.813254 82.754823) (end 133.06949 82.754823) (width 0.254) (layer "F.Cu") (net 1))
 (segment (start 110.6932 113.3348) (end 110.654665 113.373335) (width 0.254) (layer "F.Cu") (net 1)))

